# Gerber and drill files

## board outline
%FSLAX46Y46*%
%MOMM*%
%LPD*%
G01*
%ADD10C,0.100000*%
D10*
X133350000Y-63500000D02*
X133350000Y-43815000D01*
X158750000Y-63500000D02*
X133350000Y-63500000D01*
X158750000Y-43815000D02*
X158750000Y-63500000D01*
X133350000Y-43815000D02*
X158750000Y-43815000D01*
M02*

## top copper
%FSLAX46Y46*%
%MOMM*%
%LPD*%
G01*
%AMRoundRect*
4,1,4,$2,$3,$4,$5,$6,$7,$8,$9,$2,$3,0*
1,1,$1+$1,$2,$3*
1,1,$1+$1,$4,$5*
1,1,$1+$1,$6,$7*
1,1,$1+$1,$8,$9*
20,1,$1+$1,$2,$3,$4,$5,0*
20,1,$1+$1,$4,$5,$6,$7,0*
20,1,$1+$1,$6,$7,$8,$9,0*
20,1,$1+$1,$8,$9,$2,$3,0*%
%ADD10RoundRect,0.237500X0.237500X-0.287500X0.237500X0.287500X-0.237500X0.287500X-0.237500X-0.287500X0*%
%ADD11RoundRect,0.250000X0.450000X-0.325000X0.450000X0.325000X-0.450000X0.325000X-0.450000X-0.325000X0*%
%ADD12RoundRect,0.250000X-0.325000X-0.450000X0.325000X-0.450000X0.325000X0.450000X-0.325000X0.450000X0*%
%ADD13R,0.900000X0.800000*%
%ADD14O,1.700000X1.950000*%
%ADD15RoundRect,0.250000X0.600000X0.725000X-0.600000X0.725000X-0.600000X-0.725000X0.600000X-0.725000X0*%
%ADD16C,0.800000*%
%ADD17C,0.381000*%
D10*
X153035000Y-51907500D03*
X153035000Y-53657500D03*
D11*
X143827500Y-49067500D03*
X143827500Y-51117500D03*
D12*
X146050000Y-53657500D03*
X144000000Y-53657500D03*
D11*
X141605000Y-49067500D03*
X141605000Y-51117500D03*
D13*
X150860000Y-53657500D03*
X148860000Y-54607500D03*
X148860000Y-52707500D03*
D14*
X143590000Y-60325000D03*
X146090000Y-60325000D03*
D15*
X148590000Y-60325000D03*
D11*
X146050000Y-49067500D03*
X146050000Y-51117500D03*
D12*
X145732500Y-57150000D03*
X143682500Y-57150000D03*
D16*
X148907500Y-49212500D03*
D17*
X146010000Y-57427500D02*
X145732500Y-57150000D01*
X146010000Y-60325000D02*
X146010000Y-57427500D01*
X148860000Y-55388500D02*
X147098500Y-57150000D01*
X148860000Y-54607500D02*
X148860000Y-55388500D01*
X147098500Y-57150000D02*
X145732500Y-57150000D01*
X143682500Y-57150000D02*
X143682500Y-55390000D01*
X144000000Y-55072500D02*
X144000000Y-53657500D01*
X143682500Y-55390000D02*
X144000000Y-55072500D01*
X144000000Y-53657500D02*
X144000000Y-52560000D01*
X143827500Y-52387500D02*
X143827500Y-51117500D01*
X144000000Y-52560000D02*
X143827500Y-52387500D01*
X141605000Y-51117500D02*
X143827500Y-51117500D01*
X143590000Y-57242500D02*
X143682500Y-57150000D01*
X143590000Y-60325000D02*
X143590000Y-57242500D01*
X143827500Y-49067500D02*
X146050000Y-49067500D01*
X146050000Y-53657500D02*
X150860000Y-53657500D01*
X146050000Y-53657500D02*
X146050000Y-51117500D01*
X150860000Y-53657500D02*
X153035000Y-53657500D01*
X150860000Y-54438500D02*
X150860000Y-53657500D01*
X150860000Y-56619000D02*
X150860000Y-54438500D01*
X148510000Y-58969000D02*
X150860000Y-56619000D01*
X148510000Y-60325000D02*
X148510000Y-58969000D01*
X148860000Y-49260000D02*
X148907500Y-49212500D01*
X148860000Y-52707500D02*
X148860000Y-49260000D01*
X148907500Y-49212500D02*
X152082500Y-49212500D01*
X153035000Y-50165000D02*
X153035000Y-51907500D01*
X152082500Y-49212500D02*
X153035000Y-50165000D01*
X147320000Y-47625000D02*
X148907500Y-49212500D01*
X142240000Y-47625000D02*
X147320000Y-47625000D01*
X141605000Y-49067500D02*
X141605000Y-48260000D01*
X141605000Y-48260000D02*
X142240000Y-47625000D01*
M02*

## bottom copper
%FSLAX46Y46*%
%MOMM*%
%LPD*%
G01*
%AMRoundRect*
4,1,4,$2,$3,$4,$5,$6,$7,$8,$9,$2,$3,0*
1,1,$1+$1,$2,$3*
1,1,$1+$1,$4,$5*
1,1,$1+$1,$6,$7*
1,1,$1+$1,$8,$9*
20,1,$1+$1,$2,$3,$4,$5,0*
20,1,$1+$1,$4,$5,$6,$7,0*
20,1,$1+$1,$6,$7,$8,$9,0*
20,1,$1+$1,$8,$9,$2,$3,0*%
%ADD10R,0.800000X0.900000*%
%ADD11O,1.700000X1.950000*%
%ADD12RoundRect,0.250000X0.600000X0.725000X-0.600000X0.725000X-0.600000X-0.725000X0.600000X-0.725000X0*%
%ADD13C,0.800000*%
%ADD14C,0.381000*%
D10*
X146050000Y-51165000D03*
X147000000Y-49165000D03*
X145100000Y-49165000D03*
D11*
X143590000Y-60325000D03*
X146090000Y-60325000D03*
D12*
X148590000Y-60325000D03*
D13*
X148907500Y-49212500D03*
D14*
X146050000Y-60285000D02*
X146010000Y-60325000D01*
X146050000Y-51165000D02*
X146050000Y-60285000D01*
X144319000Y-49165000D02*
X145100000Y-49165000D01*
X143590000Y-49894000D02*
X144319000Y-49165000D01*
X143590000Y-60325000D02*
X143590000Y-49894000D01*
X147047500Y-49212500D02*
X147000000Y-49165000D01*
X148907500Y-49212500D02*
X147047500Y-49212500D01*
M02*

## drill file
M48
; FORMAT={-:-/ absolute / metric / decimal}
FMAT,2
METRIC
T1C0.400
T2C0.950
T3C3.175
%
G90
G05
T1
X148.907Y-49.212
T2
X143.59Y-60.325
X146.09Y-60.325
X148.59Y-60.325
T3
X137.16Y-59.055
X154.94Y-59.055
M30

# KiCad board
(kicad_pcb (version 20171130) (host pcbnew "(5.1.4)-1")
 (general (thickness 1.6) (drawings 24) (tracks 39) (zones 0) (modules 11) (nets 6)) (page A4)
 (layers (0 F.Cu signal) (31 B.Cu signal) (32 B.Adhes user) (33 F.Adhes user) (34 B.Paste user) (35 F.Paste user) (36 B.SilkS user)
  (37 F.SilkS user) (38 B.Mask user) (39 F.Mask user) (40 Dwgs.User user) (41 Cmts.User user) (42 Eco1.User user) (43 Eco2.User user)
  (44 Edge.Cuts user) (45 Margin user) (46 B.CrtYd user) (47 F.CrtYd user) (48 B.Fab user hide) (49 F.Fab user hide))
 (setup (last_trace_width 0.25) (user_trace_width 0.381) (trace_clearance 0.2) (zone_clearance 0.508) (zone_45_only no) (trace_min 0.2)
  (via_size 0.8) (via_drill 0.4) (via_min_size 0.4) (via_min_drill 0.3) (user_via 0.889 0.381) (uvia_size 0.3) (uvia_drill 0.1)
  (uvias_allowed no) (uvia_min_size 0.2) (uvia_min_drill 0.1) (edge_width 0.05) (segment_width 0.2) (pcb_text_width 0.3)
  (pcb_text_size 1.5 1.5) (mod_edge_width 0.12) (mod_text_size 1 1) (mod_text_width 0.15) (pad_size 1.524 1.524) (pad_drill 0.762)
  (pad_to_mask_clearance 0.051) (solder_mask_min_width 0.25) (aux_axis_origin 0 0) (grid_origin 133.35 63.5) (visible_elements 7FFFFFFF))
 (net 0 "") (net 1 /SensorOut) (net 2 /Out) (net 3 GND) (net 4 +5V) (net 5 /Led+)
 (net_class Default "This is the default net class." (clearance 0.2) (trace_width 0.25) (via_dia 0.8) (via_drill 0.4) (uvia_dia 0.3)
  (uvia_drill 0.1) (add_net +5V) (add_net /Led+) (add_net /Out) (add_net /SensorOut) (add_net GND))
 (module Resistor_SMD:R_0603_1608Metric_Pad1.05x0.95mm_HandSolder (layer F.Cu) (at 153.035 52.7825 90)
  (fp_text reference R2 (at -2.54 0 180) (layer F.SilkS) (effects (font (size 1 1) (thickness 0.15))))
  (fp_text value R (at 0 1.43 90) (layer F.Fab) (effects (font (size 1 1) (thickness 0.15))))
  (pad 2 smd roundrect (at 0.875 0 90) (size 1.05 0.95) (layers F.Cu F.Paste F.Mask) (roundrect_rratio 0.25) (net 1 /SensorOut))
  (pad 1 smd roundrect (at -0.875 0 90) (size 1.05 0.95) (layers F.Cu F.Paste F.Mask) (roundrect_rratio 0.25) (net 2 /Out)))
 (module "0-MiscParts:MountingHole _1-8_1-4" (layer F.Cu) (at 154.94 59.055)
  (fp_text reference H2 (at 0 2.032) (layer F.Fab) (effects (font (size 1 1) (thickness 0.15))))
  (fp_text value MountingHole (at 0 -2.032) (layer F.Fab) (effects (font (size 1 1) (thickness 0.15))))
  (pad "" np_thru_hole circle (at 0 0) (size 3.175 3.175) (drill 3.175) (layers *.Cu *.Mask)))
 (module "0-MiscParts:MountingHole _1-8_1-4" (layer F.Cu) (at 137.16 59.055)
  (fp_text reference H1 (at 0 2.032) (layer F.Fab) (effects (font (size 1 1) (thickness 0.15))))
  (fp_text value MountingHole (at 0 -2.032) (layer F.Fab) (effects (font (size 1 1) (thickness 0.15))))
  (pad "" np_thru_hole circle (at 0 0) (size 3.175 3.175) (drill 3.175) (layers *.Cu *.Mask)))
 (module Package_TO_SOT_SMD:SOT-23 (layer B.Cu) (at 146.05 50.165 270)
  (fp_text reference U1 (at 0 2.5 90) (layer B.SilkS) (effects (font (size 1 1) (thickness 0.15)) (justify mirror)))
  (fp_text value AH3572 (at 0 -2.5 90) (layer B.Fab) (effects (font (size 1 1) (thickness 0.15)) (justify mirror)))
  (pad 3 smd rect (at 1 0 270) (size 0.9 0.8) (layers B.Cu B.Paste B.Mask) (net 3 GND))
  (pad 2 smd rect (at -1 -0.95 270) (size 0.9 0.8) (layers B.Cu B.Paste B.Mask) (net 1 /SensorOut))
  (pad 1 smd rect (at -1 0.95 270) (size 0.9 0.8) (layers B.Cu B.Paste B.Mask) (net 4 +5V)))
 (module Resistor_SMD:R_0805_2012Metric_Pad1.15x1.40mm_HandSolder (layer F.Cu) (at 143.8275 50.0925 90)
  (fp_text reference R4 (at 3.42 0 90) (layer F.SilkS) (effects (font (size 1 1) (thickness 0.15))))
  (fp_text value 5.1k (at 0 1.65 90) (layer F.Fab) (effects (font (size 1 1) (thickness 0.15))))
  (pad 2 smd roundrect (at 1.025 0 90) (size 1.15 1.4) (layers F.Cu F.Paste F.Mask) (roundrect_rratio 0.217391) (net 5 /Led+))
  (pad 1 smd roundrect (at -1.025 0 90) (size 1.15 1.4) (layers F.Cu F.Paste F.Mask) (roundrect_rratio 0.217391) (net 4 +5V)))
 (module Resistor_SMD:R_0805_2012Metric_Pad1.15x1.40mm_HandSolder (layer F.Cu) (at 145.025 53.6575)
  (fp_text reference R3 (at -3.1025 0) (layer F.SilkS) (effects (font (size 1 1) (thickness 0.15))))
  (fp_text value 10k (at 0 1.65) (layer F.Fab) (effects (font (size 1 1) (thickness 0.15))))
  (pad 2 smd roundrect (at 1.025 0) (size 1.15 1.4) (layers F.Cu F.Paste F.Mask) (roundrect_rratio 0.217391) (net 2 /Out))
  (pad 1 smd roundrect (at -1.025 0) (size 1.15 1.4) (layers F.Cu F.Paste F.Mask) (roundrect_rratio 0.217391) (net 4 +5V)))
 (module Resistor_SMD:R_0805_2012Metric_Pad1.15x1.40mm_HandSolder (layer F.Cu) (at 141.605 50.0925 90)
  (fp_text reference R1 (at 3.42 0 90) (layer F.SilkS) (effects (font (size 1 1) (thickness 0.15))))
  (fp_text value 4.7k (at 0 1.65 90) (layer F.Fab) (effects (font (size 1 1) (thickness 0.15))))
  (pad 2 smd roundrect (at 1.025 0 90) (size 1.15 1.4) (layers F.Cu F.Paste F.Mask) (roundrect_rratio 0.217391) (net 1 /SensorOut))
  (pad 1 smd roundrect (at -1.025 0 90) (size 1.15 1.4) (layers F.Cu F.Paste F.Mask) (roundrect_rratio 0.217391) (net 4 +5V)))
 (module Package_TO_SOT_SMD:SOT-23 (layer F.Cu) (at 149.86 53.6575)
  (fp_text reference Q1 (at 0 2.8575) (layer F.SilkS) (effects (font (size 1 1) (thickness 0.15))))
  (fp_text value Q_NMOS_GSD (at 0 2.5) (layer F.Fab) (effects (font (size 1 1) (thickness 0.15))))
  (pad 3 smd rect (at 1 0) (size 0.9 0.8) (layers F.Cu F.Paste F.Mask) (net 2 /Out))
  (pad 2 smd rect (at -1 0.95) (size 0.9 0.8) (layers F.Cu F.Paste F.Mask) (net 3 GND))
  (pad 1 smd rect (at -1 -0.95) (size 0.9 0.8) (layers F.Cu F.Paste F.Mask) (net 1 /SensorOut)))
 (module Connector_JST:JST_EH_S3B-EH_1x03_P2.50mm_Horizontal (layer F.Cu) (at 148.59 60.325 180)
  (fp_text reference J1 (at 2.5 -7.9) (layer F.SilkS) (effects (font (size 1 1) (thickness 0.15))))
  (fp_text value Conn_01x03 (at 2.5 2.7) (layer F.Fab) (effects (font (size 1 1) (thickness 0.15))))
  (pad 3 thru_hole oval (at 5 0 180) (size 1.7 1.95) (drill 0.95) (layers *.Cu *.Mask) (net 4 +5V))
  (pad 2 thru_hole oval (at 2.5 0 180) (size 1.7 1.95) (drill 0.95) (layers *.Cu *.Mask) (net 3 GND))
  (pad 1 thru_hole roundrect (at 0 0 180) (size 1.7 1.95) (drill 0.95) (layers *.Cu *.Mask) (roundrect_rratio 0.147059) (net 2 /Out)))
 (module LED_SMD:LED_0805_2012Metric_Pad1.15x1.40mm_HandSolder (layer F.Cu) (at 146.05 50.0925 90)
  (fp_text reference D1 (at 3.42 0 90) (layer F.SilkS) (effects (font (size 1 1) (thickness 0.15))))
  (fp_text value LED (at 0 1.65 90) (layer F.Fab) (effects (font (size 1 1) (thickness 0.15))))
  (pad 2 smd roundrect (at 1.025 0 90) (size 1.15 1.4) (layers F.Cu F.Paste F.Mask) (roundrect_rratio 0.217391) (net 5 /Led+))
  (pad 1 smd roundrect (at -1.025 0 90) (size 1.15 1.4) (layers F.Cu F.Paste F.Mask) (roundrect_rratio 0.217391) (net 2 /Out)))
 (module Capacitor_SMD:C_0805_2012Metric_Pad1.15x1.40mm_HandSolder (layer F.Cu) (at 144.7075 57.15)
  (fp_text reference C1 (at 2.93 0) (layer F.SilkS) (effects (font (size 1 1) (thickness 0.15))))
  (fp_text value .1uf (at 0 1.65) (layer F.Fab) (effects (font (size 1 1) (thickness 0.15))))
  (pad 2 smd roundrect (at 1.025 0) (size 1.15 1.4) (layers F.Cu F.Paste F.Mask) (roundrect_rratio 0.217391) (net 3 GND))
  (pad 1 smd roundrect (at -1.025 0) (size 1.15 1.4) (layers F.Cu F.Paste F.Mask) (roundrect_rratio 0.217391) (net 4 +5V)))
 (gr_line (start 133.35 63.5) (end 133.35 43.815) (layer Edge.Cuts) (width 0.1))
 (gr_line (start 158.75 63.5) (end 133.35 63.5) (layer Edge.Cuts) (width 0.1))
 (gr_line (start 158.75 43.815) (end 158.75 63.5) (layer Edge.Cuts) (width 0.1))
 (gr_line (start 133.35 43.815) (end 158.75 43.815) (layer Edge.Cuts) (width 0.1))
 (segment (start 146.01 57.4275) (end 145.7325 57.15) (width 0.381) (layer F.Cu) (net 3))
 (segment (start 146.01 60.325) (end 146.01 57.4275) (width 0.381) (layer F.Cu) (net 3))
 (segment (start 148.86 55.3885) (end 147.0985 57.15) (width 0.381) (layer F.Cu) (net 3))
 (segment (start 148.86 54.6075) (end 148.86 55.3885) (width 0.381) (layer F.Cu) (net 3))
 (segment (start 147.0985 57.15) (end 145.7325 57.15) (width 0.381) (layer F.Cu) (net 3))
 (segment (start 146.05 60.285) (end 146.01 60.325) (width 0.381) (layer B.Cu) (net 3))
 (segment (start 146.05 51.165) (end 146.05 60.285) (width 0.381) (layer B.Cu) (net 3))
 (segment (start 143.6825 57.15) (end 143.6825 55.39) (width 0.381) (layer F.Cu) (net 4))
 (segment (start 144 55.0725) (end 144 53.6575) (width 0.381) (layer F.Cu) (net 4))
 (segment (start 143.6825 55.39) (end 144 55.0725) (width 0.381) (layer F.Cu) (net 4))
 (segment (start 144 53.6575) (end 144 52.56) (width 0.381) (layer F.Cu) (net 4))
 (segment (start 143.8275 52.3875) (end 143.8275 51.1175) (width 0.381) (layer F.Cu) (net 4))
 (segment (start 144 52.56) (end 143.8275 52.3875) (width 0.381) (layer F.Cu) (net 4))
 (segment (start 141.605 51.1175) (end 143.8275 51.1175) (width 0.381) (layer F.Cu) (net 4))
 (segment (start 144.319 49.165) (end 145.1 49.165) (width 0.381) (layer B.Cu) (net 4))
 (segment (start 143.59 49.894) (end 144.319 49.165) (width 0.381) (layer B.Cu) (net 4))
 (segment (start 143.59 60.325) (end 143.59 49.894) (width 0.381) (layer B.Cu) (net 4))
 (segment (start 143.59 57.2425) (end 143.6825 57.15) (width 0.381) (layer F.Cu) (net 4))
 (segment (start 143.59 60.325) (end 143.59 57.2425) (width 0.381) (layer F.Cu) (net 4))
 (segment (start 143.8275 49.0675) (end 146.05 49.0675) (width 0.381) (layer F.Cu) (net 5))
 (segment (start 146.05 53.6575) (end 150.86 53.6575) (width 0.381) (layer F.Cu) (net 2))
 (segment (start 146.05 53.6575) (end 146.05 51.1175) (width 0.381) (layer F.Cu) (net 2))
 (segment (start 150.86 53.6575) (end 153.035 53.6575) (width 0.381) (layer F.Cu) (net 2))
 (segment (start 150.86 54.4385) (end 150.86 53.6575) (width 0.381) (layer F.Cu) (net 2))
 (segment (start 150.86 56.619) (end 150.86 54.4385) (width 0.381) (layer F.Cu) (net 2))
 (segment (start 148.51 58.969) (end 150.86 56.619) (width 0.381) (layer F.Cu) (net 2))
 (segment (start 148.51 60.325) (end 148.51 58.969) (width 0.381) (layer F.Cu) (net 2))
 (via (at 148.9075 49.2125) (size 0.8) (drill 0.4) (layers F.Cu B.Cu) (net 1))
 (segment (start 148.86 49.26) (end 148.9075 49.2125) (width 0.381) (layer F.Cu) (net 1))
 (segment (start 148.86 52.7075) (end 148.86 49.26) (width 0.381) (layer F.Cu) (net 1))
 (segment (start 148.9075 49.2125) (end 152.0825 49.2125) (width 0.381) (layer F.Cu) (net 1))
 (segment (start 153.035 50.165) (end 153.035 51.9075) (width 0.381) (layer F.Cu) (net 1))
 (segment (start 152.0825 49.2125) (end 153.035 50.165) (width 0.381) (layer F.Cu) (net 1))
 (segment (start 147.0475 49.2125) (end 147 49.165) (width 0.381) (layer B.Cu) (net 1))
 (segment (start 148.9075 49.2125) (end 147.0475 49.2125) (width 0.381) (layer B.Cu) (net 1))
 (segment (start 147.32 47.625) (end 148.9075 49.2125) (width 0.381) (layer F.Cu) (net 1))
 (segment (start 142.24 47.625) (end 147.32 47.625) (width 0.381) (layer F.Cu) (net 1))
 (segment (start 141.605 49.0675) (end 141.605 48.26) (width 0.381) (layer F.Cu) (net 1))
 (segment (start 141.605 48.26) (end 142.24 47.625) (width 0.381) (layer F.Cu) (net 1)))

